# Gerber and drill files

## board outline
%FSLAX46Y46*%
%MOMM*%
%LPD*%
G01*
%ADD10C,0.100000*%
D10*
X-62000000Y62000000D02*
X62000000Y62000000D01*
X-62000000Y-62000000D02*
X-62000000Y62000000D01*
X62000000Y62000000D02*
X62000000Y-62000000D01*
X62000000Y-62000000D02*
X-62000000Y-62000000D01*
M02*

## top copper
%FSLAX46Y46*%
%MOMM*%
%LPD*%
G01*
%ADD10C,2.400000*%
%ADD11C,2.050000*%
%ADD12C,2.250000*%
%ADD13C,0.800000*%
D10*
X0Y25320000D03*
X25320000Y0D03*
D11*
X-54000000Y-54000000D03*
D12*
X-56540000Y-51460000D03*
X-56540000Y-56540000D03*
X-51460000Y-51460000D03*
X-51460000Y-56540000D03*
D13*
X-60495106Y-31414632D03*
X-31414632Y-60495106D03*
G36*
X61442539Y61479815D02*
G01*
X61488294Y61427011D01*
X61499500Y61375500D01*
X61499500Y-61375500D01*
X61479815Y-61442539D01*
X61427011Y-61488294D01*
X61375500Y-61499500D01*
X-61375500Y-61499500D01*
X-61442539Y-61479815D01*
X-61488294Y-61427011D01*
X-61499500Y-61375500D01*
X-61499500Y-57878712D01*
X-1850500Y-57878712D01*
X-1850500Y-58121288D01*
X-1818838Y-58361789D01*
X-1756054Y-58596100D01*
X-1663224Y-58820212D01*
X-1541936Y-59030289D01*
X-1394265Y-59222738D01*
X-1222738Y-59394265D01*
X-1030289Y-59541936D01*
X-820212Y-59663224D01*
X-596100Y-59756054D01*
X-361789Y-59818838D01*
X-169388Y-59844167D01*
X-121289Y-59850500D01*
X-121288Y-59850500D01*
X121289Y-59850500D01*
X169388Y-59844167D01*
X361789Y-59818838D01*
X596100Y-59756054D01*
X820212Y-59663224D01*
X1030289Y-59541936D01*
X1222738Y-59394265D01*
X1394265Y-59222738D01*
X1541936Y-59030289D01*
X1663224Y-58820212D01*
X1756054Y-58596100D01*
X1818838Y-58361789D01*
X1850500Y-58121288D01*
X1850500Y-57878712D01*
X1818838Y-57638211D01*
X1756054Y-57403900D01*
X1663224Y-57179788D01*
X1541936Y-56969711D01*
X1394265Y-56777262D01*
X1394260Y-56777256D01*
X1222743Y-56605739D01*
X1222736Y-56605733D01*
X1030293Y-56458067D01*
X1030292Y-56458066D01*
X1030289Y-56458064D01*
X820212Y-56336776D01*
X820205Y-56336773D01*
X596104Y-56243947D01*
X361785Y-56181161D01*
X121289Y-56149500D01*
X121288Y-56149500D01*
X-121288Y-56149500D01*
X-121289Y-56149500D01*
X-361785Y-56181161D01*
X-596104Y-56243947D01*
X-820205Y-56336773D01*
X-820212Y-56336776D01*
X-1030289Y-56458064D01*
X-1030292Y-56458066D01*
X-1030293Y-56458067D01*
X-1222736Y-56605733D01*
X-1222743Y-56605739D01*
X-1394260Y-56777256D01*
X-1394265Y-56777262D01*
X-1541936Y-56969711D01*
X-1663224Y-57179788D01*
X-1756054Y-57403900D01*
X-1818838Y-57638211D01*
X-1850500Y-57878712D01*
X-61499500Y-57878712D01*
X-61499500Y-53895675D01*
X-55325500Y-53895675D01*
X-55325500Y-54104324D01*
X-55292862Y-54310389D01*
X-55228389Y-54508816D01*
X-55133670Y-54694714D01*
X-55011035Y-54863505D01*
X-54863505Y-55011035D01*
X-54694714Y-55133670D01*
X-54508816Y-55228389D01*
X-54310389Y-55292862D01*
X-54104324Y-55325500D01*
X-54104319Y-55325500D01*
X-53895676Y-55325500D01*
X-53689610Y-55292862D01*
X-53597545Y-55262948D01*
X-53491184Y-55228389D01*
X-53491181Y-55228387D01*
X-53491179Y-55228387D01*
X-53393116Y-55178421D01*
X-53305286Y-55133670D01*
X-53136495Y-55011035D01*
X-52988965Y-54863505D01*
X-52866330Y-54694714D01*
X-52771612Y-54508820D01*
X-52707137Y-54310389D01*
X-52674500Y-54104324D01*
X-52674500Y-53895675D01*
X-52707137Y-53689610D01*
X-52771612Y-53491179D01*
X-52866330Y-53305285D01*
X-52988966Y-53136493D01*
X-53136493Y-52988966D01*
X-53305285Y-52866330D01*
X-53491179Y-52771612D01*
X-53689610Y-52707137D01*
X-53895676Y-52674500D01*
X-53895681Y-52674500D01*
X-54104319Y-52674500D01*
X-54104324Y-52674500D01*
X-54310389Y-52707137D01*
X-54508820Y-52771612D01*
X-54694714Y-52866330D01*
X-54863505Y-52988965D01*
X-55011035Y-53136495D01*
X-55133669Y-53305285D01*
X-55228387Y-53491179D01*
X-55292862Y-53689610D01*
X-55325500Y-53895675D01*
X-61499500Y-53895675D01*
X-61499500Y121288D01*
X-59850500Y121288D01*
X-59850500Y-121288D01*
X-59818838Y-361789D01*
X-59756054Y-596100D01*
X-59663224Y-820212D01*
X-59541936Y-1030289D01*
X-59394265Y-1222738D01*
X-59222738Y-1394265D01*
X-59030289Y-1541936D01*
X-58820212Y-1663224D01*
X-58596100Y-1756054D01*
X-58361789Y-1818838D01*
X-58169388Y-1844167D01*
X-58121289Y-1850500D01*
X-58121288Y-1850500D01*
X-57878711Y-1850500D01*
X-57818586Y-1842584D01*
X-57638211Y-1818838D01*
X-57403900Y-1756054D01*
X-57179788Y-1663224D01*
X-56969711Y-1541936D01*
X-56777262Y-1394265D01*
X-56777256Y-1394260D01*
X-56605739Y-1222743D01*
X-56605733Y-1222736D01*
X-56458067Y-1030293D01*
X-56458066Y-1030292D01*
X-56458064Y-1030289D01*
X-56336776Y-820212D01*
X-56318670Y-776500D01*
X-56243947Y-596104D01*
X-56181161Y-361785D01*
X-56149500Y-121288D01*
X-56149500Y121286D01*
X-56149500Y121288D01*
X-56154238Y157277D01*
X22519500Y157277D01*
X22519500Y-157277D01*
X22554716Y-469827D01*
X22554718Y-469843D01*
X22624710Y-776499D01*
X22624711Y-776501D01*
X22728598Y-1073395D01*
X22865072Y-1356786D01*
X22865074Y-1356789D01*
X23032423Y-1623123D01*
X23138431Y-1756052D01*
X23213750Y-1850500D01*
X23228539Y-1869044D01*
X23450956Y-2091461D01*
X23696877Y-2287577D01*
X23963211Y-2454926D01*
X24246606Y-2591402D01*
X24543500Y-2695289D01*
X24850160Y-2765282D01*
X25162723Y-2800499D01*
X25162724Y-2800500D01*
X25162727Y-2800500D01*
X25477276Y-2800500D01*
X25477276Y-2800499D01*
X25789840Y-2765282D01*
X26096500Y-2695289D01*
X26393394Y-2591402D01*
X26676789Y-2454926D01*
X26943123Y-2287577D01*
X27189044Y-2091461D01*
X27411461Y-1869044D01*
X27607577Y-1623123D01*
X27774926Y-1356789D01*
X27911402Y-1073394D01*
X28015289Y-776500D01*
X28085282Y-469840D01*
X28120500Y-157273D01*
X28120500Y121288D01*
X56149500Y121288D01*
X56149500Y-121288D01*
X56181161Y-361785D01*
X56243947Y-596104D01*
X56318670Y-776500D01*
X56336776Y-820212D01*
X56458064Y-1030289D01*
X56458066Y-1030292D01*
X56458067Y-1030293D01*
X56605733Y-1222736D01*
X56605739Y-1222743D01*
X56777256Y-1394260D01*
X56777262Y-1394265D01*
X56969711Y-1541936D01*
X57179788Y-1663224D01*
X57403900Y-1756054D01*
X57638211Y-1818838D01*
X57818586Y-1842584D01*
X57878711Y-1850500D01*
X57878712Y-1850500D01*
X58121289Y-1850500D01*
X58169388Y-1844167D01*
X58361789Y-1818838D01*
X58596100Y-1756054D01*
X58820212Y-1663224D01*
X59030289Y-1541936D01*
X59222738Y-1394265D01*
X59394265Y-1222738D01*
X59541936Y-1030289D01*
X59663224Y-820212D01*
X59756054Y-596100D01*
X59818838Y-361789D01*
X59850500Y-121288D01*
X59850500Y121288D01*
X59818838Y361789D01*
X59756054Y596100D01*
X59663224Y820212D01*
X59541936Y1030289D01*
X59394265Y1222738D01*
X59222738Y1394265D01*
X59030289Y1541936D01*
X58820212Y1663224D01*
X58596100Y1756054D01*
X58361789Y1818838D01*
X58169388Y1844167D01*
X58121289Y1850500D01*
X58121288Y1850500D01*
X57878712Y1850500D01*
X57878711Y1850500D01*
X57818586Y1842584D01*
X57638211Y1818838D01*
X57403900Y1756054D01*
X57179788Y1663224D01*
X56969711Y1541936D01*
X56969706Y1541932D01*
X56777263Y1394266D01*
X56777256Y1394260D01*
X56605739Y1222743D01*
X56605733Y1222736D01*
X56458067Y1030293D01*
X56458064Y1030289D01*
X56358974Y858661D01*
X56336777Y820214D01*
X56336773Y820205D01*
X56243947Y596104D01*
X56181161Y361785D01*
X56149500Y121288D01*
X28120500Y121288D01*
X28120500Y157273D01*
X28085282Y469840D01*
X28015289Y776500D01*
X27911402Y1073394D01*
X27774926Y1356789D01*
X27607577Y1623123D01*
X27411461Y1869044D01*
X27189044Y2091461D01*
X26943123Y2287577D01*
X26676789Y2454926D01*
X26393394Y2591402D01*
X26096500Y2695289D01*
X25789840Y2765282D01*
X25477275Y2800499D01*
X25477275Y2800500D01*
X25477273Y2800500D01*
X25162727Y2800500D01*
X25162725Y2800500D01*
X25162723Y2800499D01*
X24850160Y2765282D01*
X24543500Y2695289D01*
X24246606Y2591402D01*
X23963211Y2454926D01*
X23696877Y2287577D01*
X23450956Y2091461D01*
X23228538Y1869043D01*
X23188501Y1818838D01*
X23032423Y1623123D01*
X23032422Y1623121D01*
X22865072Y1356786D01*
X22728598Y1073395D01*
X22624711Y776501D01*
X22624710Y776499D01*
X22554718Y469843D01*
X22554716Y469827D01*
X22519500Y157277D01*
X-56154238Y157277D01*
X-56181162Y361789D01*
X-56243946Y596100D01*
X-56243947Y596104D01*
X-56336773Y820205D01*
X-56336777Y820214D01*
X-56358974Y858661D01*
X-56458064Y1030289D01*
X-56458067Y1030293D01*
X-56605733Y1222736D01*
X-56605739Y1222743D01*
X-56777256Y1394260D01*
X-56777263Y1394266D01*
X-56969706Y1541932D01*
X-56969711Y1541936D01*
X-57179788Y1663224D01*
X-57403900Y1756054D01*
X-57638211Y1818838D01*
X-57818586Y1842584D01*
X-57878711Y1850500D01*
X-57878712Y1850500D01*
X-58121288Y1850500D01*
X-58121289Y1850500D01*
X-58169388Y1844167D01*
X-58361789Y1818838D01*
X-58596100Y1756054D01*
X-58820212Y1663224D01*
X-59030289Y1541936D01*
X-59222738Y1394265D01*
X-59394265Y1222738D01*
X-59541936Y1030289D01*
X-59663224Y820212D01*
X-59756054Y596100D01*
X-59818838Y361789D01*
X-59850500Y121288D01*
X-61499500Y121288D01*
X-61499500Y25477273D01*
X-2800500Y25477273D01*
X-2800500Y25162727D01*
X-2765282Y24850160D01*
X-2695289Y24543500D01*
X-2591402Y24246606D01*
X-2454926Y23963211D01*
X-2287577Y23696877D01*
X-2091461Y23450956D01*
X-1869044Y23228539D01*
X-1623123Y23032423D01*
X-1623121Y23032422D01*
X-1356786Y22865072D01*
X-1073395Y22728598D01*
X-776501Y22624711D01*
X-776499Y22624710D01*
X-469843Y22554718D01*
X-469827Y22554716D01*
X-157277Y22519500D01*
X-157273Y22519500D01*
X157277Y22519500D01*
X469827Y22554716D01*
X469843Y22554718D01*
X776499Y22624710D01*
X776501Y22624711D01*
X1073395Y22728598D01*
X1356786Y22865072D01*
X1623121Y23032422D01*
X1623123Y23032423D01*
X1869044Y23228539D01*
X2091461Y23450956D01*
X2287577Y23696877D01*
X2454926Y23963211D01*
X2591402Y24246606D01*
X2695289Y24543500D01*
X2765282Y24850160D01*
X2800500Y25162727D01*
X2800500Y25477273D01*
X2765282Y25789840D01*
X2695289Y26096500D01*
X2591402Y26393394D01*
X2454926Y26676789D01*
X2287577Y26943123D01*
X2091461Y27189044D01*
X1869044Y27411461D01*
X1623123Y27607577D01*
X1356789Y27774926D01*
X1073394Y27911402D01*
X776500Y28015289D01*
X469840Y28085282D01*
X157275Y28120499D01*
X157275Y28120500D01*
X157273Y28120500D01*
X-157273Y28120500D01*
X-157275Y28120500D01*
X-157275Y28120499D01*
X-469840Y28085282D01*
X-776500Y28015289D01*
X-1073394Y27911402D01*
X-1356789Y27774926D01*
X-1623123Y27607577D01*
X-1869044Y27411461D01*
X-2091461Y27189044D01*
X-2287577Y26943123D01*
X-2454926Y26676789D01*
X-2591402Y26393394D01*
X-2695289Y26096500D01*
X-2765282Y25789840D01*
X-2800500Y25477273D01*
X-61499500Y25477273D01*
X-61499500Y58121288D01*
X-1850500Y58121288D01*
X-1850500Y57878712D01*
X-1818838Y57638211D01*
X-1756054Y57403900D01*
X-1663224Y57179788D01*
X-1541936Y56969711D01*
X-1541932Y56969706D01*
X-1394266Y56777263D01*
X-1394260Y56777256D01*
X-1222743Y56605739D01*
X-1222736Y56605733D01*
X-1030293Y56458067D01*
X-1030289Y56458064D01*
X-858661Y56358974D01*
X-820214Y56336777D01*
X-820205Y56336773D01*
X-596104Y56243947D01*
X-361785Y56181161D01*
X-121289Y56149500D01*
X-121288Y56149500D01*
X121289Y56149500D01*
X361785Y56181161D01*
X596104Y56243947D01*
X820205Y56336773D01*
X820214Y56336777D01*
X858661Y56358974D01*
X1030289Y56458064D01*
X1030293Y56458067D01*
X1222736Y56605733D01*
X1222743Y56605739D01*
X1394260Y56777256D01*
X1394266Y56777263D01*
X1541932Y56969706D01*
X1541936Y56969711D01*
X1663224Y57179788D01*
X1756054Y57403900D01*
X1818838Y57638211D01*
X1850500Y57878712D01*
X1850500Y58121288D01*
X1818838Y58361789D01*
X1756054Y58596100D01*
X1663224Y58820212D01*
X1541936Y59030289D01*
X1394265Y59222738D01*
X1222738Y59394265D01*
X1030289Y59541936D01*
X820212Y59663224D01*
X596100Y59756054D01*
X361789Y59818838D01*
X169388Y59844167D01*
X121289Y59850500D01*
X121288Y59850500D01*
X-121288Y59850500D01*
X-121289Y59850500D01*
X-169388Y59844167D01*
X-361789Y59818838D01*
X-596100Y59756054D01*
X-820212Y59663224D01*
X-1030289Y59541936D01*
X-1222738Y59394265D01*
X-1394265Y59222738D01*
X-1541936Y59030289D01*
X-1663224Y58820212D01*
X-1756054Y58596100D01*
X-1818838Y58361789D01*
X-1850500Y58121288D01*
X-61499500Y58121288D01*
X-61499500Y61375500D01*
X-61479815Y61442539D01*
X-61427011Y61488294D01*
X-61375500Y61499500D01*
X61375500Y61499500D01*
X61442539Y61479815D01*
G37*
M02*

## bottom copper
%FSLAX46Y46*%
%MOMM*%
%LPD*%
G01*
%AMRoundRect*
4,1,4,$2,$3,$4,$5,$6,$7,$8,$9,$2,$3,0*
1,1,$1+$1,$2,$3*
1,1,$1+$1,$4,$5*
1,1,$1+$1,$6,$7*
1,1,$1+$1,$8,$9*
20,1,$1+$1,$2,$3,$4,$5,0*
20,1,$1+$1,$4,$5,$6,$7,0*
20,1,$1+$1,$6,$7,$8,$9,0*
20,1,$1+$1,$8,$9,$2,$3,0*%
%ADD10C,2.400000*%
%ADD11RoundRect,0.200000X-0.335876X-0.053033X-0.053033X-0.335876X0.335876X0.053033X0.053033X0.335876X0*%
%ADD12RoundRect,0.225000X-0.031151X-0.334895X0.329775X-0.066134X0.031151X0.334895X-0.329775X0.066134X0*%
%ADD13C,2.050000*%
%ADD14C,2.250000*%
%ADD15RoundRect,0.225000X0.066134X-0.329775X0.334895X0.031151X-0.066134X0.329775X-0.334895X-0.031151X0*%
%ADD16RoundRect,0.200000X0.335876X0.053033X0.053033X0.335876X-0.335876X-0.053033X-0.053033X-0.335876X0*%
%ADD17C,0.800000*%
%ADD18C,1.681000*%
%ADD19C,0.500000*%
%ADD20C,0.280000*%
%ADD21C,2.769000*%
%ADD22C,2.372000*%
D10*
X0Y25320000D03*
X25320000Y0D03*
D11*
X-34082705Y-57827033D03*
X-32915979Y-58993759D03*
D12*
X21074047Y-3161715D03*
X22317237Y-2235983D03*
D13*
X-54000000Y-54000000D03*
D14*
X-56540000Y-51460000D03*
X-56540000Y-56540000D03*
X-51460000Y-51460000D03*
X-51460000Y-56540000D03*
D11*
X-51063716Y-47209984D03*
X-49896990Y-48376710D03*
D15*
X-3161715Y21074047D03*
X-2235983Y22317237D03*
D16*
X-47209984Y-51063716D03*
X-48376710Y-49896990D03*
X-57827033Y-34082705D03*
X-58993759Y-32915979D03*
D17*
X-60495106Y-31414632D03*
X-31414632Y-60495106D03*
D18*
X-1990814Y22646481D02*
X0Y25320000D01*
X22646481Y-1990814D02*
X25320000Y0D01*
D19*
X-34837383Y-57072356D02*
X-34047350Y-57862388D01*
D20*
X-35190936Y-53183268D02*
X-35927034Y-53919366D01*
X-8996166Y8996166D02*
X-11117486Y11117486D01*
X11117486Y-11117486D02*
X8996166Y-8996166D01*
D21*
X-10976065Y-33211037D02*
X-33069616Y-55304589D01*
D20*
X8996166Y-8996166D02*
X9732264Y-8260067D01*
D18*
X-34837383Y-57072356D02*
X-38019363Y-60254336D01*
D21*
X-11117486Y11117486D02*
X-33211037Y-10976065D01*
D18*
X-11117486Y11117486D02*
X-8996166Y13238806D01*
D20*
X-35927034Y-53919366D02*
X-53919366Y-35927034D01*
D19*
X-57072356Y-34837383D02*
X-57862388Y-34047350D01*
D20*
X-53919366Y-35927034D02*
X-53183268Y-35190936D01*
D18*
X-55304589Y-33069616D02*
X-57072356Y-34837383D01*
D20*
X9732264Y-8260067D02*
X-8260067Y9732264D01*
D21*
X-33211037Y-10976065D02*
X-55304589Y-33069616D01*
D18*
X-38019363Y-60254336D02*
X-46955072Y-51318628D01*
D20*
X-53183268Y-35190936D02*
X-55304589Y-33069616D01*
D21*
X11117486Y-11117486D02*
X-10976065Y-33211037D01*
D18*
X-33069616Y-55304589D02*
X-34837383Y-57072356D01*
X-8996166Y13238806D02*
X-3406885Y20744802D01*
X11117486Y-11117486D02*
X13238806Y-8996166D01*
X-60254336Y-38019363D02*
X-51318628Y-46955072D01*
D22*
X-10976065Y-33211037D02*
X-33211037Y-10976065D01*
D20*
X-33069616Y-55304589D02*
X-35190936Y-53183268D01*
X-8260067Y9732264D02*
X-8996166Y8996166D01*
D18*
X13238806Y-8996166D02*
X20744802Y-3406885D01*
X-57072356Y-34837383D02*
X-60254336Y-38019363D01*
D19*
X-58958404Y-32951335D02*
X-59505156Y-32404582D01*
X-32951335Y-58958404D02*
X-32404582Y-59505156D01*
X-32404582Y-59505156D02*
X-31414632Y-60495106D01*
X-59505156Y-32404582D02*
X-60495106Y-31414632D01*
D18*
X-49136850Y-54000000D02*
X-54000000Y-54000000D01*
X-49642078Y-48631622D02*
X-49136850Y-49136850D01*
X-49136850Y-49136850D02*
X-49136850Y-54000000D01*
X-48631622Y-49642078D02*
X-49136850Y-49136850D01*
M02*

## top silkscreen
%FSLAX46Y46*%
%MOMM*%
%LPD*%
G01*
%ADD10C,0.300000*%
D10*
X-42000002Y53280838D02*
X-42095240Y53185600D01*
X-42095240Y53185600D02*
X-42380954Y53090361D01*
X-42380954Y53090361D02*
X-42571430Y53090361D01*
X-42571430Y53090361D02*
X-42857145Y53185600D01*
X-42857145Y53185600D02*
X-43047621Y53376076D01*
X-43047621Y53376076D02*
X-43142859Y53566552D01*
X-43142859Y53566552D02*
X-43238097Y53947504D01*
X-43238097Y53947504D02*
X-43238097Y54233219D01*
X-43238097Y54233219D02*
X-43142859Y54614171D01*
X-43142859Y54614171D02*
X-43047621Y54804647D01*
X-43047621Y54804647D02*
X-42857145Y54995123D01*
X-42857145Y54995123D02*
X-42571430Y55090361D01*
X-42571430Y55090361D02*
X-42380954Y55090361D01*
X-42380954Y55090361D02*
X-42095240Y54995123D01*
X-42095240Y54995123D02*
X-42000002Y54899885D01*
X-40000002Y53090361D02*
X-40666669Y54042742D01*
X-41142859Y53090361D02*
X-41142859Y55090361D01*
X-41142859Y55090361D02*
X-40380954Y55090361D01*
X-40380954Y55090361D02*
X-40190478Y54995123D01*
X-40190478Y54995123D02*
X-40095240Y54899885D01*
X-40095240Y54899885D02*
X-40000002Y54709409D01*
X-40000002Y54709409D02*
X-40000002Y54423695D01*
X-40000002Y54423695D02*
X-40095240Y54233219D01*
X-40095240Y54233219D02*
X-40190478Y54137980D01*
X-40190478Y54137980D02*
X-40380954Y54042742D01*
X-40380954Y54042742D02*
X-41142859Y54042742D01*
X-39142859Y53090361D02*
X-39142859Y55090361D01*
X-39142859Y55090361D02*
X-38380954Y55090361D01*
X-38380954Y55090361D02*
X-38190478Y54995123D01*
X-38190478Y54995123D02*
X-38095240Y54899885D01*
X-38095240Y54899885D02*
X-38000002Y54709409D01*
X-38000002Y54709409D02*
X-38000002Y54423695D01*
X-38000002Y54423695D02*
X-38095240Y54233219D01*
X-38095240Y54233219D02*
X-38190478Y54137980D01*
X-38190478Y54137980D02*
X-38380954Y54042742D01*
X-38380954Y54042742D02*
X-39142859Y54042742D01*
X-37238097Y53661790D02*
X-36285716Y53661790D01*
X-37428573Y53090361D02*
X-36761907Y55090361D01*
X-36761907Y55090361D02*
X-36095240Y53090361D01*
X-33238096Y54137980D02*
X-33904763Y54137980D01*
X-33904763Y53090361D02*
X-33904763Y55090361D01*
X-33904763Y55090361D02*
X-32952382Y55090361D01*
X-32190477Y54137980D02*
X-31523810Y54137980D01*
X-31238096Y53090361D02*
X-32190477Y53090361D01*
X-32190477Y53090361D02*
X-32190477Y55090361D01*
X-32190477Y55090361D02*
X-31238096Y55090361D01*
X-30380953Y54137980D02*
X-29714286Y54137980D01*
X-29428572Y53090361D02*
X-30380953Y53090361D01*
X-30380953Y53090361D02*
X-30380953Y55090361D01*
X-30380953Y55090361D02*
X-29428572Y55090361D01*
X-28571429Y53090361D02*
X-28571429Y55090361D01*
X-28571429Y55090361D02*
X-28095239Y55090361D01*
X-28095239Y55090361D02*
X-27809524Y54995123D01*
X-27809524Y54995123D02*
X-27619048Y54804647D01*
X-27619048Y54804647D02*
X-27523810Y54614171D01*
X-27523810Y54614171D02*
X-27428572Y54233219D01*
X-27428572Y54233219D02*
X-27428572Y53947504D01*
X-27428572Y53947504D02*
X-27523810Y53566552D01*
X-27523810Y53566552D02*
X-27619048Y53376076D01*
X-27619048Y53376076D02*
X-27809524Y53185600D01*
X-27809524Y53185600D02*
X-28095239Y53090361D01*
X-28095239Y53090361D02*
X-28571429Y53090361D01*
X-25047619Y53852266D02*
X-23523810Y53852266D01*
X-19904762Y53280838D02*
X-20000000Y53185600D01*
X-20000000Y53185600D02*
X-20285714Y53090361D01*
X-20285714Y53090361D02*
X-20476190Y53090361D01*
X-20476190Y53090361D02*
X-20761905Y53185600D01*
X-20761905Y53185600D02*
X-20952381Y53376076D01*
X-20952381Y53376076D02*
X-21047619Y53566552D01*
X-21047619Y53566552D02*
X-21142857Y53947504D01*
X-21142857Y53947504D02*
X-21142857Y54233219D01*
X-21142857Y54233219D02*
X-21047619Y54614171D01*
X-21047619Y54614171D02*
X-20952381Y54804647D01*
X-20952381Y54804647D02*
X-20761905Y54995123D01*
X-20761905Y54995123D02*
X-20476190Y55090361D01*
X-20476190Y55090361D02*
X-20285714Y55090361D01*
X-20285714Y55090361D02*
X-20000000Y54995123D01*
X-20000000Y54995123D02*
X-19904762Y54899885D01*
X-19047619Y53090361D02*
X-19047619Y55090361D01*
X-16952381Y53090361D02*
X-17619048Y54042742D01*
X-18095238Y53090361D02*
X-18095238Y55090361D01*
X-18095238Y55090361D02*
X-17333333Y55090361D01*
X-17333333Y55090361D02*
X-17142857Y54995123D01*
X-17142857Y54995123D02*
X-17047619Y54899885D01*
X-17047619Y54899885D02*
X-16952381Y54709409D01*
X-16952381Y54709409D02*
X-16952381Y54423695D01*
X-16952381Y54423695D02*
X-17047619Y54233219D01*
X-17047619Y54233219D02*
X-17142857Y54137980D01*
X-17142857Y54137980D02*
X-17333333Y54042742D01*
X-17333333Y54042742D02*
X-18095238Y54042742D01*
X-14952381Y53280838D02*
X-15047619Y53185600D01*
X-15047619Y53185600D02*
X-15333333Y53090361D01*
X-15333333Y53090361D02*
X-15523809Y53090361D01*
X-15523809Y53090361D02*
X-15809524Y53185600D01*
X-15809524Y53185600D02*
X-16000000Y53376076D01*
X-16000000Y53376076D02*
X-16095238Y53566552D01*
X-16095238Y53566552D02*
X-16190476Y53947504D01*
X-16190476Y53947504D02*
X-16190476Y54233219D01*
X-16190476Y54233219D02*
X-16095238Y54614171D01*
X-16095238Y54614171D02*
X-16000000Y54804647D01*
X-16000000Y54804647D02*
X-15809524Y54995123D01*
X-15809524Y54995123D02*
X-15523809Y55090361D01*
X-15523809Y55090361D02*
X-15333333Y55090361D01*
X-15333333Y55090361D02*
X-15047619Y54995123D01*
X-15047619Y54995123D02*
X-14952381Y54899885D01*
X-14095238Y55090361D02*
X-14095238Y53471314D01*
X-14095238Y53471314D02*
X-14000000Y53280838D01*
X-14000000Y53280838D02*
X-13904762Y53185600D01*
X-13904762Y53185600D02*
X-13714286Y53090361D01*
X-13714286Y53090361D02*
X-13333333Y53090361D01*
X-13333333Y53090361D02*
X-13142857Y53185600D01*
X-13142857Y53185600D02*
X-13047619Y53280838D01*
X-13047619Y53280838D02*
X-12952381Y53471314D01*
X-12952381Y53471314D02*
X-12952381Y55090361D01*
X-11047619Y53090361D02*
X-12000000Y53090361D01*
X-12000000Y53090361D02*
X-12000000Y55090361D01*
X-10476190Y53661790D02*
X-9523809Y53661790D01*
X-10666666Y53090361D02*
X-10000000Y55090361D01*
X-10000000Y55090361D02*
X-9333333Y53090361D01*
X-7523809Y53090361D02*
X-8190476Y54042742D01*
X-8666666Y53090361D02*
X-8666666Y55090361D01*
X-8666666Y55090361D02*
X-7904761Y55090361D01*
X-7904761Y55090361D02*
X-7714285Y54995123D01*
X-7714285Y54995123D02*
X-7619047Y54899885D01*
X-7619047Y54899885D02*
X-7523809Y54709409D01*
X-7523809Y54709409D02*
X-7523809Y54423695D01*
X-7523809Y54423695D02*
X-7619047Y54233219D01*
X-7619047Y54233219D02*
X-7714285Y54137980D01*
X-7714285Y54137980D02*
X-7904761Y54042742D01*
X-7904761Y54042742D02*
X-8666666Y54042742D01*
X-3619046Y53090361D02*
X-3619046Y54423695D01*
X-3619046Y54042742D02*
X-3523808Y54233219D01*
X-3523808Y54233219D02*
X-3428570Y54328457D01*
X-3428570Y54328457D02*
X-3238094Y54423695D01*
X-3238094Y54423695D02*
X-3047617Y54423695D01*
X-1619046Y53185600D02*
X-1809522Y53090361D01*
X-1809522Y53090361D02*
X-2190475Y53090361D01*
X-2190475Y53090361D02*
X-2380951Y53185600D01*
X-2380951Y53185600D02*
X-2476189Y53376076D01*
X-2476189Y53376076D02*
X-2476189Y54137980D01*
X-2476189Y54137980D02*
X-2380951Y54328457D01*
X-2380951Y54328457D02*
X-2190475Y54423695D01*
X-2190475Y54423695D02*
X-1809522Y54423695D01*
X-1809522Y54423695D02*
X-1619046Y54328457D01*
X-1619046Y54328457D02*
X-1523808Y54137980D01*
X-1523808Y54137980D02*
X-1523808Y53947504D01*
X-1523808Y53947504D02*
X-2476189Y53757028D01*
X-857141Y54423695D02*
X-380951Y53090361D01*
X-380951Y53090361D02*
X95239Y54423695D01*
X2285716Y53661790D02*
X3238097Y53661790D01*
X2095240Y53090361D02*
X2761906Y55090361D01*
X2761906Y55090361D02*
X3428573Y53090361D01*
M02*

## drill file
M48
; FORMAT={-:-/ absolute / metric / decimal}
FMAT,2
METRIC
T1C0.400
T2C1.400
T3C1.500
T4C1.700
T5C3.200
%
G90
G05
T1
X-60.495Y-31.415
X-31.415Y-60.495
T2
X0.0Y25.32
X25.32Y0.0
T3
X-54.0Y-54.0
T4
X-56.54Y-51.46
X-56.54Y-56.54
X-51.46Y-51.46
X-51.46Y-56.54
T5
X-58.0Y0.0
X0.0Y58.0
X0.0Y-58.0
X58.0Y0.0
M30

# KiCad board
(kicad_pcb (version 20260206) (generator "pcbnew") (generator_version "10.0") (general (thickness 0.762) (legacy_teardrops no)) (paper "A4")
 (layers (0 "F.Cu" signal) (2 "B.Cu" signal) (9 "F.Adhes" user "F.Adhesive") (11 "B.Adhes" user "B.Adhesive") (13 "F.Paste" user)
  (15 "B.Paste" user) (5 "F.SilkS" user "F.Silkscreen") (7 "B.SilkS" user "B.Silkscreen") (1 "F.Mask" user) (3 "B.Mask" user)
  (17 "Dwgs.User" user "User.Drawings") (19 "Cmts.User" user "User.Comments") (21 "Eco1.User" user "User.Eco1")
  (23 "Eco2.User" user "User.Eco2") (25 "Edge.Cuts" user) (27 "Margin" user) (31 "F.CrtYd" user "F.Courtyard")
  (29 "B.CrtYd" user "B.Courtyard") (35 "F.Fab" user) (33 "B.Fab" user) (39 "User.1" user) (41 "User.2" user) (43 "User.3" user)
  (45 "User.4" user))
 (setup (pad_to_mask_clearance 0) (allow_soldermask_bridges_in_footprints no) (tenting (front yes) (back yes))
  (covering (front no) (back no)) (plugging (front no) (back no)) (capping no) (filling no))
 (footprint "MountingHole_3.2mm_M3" (layer "F.Cu") (at 0 58)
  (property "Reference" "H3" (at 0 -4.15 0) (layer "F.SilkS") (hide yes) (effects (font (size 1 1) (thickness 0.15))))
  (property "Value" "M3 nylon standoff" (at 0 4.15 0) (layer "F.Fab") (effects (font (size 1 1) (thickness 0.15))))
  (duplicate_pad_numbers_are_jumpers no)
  (pad "" np_thru_hole circle (at 0 0) (size 3.2 3.2) (drill 3.2) (layers "*.Cu" "*.Mask")))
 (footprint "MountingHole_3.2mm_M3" (layer "F.Cu") (at 58 0)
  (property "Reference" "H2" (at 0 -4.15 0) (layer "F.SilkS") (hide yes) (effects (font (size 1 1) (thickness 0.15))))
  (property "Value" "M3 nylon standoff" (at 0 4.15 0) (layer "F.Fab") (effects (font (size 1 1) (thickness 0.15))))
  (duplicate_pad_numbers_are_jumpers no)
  (pad "" np_thru_hole circle (at 0 0) (size 3.2 3.2) (drill 3.2) (layers "*.Cu" "*.Mask")))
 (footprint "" (layer "F.Cu") (at 0 -25.32)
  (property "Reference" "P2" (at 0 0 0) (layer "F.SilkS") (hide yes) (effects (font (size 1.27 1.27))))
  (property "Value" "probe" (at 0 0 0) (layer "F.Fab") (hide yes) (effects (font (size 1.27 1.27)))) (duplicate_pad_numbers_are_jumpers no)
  (pad "1" thru_hole circle (at 0 0) (size 2.4 2.4) (drill 1.4) (layers "*.Cu" "*.Mask") (remove_unused_layers no) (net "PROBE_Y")
   (clearance 1.6)))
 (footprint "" (layer "F.Cu") (at 25.32 0)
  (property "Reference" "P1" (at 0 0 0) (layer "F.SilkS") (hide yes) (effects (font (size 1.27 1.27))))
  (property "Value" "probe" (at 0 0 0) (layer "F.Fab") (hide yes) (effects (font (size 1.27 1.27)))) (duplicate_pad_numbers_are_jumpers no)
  (pad "1" thru_hole circle (at 0 0) (size 2.4 2.4) (drill 1.4) (layers "*.Cu" "*.Mask") (remove_unused_layers no) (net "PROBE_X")
   (clearance 1.6)))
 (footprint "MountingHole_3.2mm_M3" (layer "F.Cu") (at 0 -58)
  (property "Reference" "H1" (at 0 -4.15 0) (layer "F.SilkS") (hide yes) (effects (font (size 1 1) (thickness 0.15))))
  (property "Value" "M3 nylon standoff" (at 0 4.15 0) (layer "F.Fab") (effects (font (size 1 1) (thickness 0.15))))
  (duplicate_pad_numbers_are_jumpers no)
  (pad "" np_thru_hole circle (at 0 0) (size 3.2 3.2) (drill 3.2) (layers "*.Cu" "*.Mask")))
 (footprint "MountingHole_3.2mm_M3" (layer "F.Cu") (at -58 0)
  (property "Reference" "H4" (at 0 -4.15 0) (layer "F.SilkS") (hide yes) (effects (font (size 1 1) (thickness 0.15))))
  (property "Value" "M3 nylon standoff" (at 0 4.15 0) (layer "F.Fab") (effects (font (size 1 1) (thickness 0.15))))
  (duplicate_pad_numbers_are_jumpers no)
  (pad "" np_thru_hole circle (at 0 0) (size 3.2 3.2) (drill 3.2) (layers "*.Cu" "*.Mask")))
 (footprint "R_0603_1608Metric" (layer "B.Cu") (at -33.499342 58.410396 -45)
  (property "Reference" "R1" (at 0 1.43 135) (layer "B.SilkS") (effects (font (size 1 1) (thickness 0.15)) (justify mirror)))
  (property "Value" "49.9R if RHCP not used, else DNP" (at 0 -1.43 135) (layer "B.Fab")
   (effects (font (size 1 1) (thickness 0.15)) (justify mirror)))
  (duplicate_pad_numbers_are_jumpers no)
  (pad "1" smd roundrect (at -0.825 0 315) (size 0.8 0.95) (layers "B.Cu" "B.Mask" "B.Paste") (roundrect_rratio 0.25) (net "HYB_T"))
  (pad "2" smd roundrect (at 0.825 0 315) (size 0.8 0.95) (layers "B.Cu" "B.Mask" "B.Paste") (roundrect_rratio 0.25) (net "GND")))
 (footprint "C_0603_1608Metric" (layer "B.Cu") (at 21.695642 2.698849 36.67292409)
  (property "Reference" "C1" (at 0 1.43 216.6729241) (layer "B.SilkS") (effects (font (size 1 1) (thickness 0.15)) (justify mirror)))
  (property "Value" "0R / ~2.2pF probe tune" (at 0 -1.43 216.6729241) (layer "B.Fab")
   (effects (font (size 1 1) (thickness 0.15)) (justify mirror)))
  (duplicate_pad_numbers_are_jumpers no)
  (pad "1" smd roundrect (at -0.775 0 36.67292409) (size 0.9 0.95) (layers "B.Cu" "B.Mask" "B.Paste") (roundrect_rratio 0.25) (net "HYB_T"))
  (pad "2" smd roundrect (at 0.775 0 36.67292409) (size 0.9 0.95) (layers "B.Cu" "B.Mask" "B.Paste") (roundrect_rratio 0.25) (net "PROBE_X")))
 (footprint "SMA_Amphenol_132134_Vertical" (layer "B.Cu") (at -54 54)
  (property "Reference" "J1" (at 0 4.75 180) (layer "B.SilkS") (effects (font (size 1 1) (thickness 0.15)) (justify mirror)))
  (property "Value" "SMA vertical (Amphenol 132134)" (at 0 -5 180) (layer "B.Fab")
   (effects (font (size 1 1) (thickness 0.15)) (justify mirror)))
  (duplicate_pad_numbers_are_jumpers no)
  (pad "1" thru_hole circle (at 0 0) (size 2.05 2.05) (drill 1.5) (layers "*.Cu" "*.Mask") (remove_unused_layers no) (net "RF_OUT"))
  (pad "2" thru_hole circle (at -2.54 -2.54) (size 2.25 2.25) (drill 1.7) (layers "*.Cu" "*.Mask") (remove_unused_layers no) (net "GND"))
  (pad "2" thru_hole circle (at -2.54 2.54) (size 2.25 2.25) (drill 1.7) (layers "*.Cu" "*.Mask") (remove_unused_layers no) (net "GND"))
  (pad "2" thru_hole circle (at 2.54 -2.54) (size 2.25 2.25) (drill 1.7) (layers "*.Cu" "*.Mask") (remove_unused_layers no) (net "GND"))
  (pad "2" thru_hole circle (at 2.54 2.54) (size 2.25 2.25) (drill 1.7) (layers "*.Cu" "*.Mask") (remove_unused_layers no) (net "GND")))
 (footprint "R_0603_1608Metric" (layer "B.Cu") (at -50.480353 47.793347 -45)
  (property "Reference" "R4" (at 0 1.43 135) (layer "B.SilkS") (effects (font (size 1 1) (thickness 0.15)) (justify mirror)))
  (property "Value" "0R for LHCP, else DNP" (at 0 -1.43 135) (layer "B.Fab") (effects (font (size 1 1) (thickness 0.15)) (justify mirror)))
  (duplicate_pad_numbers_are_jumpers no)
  (pad "1" smd roundrect (at -0.825 0 315) (size 0.8 0.95) (layers "B.Cu" "B.Mask" "B.Paste") (roundrect_rratio 0.25) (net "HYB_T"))
  (pad "2" smd roundrect (at 0.825 0 315) (size 0.8 0.95) (layers "B.Cu" "B.Mask" "B.Paste") (roundrect_rratio 0.25) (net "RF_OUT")))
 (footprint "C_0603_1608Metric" (layer "B.Cu") (at -2.698849 -21.695642 53.32707591)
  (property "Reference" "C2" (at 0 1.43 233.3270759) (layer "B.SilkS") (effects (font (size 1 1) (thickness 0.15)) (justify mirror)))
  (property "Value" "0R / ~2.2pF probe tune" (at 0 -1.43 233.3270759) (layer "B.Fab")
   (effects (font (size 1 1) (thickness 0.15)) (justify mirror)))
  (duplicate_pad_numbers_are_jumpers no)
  (pad "1" smd roundrect (at -0.775 0 53.32707591) (size 0.9 0.95) (layers "B.Cu" "B.Mask" "B.Paste") (roundrect_rratio 0.25) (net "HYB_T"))
  (pad "2" smd roundrect (at 0.775 0 53.32707591) (size 0.9 0.95) (layers "B.Cu" "B.Mask" "B.Paste") (roundrect_rratio 0.25) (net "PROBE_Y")))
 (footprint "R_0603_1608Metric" (layer "B.Cu") (at -47.793347 50.480353 135)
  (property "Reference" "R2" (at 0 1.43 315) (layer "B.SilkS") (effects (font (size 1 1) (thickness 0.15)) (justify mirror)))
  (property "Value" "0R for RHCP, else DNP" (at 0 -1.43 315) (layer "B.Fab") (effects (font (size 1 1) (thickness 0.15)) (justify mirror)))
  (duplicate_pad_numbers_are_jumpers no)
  (pad "1" smd roundrect (at -0.825 0 135) (size 0.8 0.95) (layers "B.Cu" "B.Mask" "B.Paste") (roundrect_rratio 0.25) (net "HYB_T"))
  (pad "2" smd roundrect (at 0.825 0 135) (size 0.8 0.95) (layers "B.Cu" "B.Mask" "B.Paste") (roundrect_rratio 0.25) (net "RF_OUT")))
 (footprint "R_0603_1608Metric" (layer "B.Cu") (at -58.410396 33.499342 135)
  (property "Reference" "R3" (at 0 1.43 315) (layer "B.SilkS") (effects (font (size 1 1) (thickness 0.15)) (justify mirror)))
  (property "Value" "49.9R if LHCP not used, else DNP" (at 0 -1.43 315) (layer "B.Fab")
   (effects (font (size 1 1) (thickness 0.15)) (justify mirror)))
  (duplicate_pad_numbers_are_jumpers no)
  (pad "1" smd roundrect (at -0.825 0 135) (size 0.8 0.95) (layers "B.Cu" "B.Mask" "B.Paste") (roundrect_rratio 0.25) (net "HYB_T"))
  (pad "2" smd roundrect (at 0.825 0 135) (size 0.8 0.95) (layers "B.Cu" "B.Mask" "B.Paste") (roundrect_rratio 0.25) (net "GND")))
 (gr_line (start -62 -62) (end 62 -62) (stroke (width 0.1) (type default)) (layer "Edge.Cuts"))
 (gr_line (start -62 62) (end -62 -62) (stroke (width 0.1) (type default)) (layer "Edge.Cuts"))
 (gr_line (start 62 -62) (end 62 62) (stroke (width 0.1) (type default)) (layer "Edge.Cuts"))
 (gr_line (start 62 62) (end -62 62) (stroke (width 0.1) (type default)) (layer "Edge.Cuts"))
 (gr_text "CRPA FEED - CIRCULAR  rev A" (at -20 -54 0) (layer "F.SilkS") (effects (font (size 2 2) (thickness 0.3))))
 (segment (start -1.990814 -22.646481) (end 0 -25.32) (width 1.681) (layer "B.Cu") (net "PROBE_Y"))
 (segment (start 22.646481 1.990814) (end 25.32 0) (width 1.681) (layer "B.Cu") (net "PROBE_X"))
 (segment (start -34.837383 57.072356) (end -34.04735 57.862388) (width 0.5) (layer "B.Cu") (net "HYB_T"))
 (segment (start -35.190936 53.183268) (end -35.927034 53.919366) (width 0.28) (layer "B.Cu") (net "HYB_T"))
 (segment (start -8.996166 -8.996166) (end -11.117486 -11.117486) (width 0.28) (layer "B.Cu") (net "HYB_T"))
 (segment (start 11.117486 11.117486) (end 8.996166 8.996166) (width 0.28) (layer "B.Cu") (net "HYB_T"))
 (segment (start -10.976065 33.211037) (end -33.069616 55.304589) (width 2.769) (layer "B.Cu") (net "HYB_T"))
 (segment (start 8.996166 8.996166) (end 9.732264 8.260067) (width 0.28) (layer "B.Cu") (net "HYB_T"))
 (segment (start -34.837383 57.072356) (end -38.019363 60.254336) (width 1.681) (layer "B.Cu") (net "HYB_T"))
 (segment (start -11.117486 -11.117486) (end -33.211037 10.976065) (width 2.769) (layer "B.Cu") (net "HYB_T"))
 (segment (start -11.117486 -11.117486) (end -8.996166 -13.238806) (width 1.681) (layer "B.Cu") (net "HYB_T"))
 (segment (start -35.927034 53.919366) (end -53.919366 35.927034) (width 0.28) (layer "B.Cu") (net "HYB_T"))
 (segment (start -57.072356 34.837383) (end -57.862388 34.04735) (width 0.5) (layer "B.Cu") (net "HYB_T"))
 (segment (start -53.919366 35.927034) (end -53.183268 35.190936) (width 0.28) (layer "B.Cu") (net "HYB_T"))
 (segment (start -55.304589 33.069616) (end -57.072356 34.837383) (width 1.681) (layer "B.Cu") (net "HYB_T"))
 (segment (start 9.732264 8.260067) (end -8.260067 -9.732264) (width 0.28) (layer "B.Cu") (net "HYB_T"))
 (segment (start -33.211037 10.976065) (end -55.304589 33.069616) (width 2.769) (layer "B.Cu") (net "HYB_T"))
 (segment (start -38.019363 60.254336) (end -46.955072 51.318628) (width 1.681) (layer "B.Cu") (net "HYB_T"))
 (segment (start -53.183268 35.190936) (end -55.304589 33.069616) (width 0.28) (layer "B.Cu") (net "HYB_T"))
 (segment (start 11.117486 11.117486) (end -10.976065 33.211037) (width 2.769) (layer "B.Cu") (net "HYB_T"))
 (segment (start -33.069616 55.304589) (end -34.837383 57.072356) (width 1.681) (layer "B.Cu") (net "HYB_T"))
 (segment (start -8.996166 -13.238806) (end -3.406885 -20.744802) (width 1.681) (layer "B.Cu") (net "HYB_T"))
 (segment (start 11.117486 11.117486) (end 13.238806 8.996166) (width 1.681) (layer "B.Cu") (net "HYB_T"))
 (segment (start -60.254336 38.019363) (end -51.318628 46.955072) (width 1.681) (layer "B.Cu") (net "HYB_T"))
 (segment (start -10.976065 33.211037) (end -33.211037 10.976065) (width 2.372) (layer "B.Cu") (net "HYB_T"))
 (segment (start -33.069616 55.304589) (end -35.190936 53.183268) (width 0.28) (layer "B.Cu") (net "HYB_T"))
 (segment (start -8.260067 -9.732264) (end -8.996166 -8.996166) (width 0.28) (layer "B.Cu") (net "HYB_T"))
 (segment (start 13.238806 8.996166) (end 20.744802 3.406885) (width 1.681) (layer "B.Cu") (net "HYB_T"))
 (segment (start -57.072356 34.837383) (end -60.254336 38.019363) (width 1.681) (layer "B.Cu") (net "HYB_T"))
 (via (at -60.495106 31.414632) (size 0.8) (drill 0.4) (layers "F.Cu" "B.Cu") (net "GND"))
 (via (at -31.414632 60.495106) (size 0.8) (drill 0.4) (layers "F.Cu" "B.Cu") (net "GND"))
 (segment (start -58.958404 32.951335) (end -59.505156 32.404582) (width 0.5) (layer "B.Cu") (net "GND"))
 (segment (start -32.951335 58.958404) (end -32.404582 59.505156) (width 0.5) (layer "B.Cu") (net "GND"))
 (segment (start -32.404582 59.505156) (end -31.414632 60.495106) (width 0.5) (layer "B.Cu") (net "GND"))
 (segment (start -59.505156 32.404582) (end -60.495106 31.414632) (width 0.5) (layer "B.Cu") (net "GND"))
 (segment (start -49.13685 54) (end -54 54) (width 1.681) (layer "B.Cu") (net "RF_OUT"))
 (segment (start -49.642078 48.631622) (end -49.13685 49.13685) (width 1.681) (layer "B.Cu") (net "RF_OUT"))
 (segment (start -49.13685 49.13685) (end -49.13685 54) (width 1.681) (layer "B.Cu") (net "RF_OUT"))
 (segment (start -48.631622 49.642078) (end -49.13685 49.13685) (width 1.681) (layer "B.Cu") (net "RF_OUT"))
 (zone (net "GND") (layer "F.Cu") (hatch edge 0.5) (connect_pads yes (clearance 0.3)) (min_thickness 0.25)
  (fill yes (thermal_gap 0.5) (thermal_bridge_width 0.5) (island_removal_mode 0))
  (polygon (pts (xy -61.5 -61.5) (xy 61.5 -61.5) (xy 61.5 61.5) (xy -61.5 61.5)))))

